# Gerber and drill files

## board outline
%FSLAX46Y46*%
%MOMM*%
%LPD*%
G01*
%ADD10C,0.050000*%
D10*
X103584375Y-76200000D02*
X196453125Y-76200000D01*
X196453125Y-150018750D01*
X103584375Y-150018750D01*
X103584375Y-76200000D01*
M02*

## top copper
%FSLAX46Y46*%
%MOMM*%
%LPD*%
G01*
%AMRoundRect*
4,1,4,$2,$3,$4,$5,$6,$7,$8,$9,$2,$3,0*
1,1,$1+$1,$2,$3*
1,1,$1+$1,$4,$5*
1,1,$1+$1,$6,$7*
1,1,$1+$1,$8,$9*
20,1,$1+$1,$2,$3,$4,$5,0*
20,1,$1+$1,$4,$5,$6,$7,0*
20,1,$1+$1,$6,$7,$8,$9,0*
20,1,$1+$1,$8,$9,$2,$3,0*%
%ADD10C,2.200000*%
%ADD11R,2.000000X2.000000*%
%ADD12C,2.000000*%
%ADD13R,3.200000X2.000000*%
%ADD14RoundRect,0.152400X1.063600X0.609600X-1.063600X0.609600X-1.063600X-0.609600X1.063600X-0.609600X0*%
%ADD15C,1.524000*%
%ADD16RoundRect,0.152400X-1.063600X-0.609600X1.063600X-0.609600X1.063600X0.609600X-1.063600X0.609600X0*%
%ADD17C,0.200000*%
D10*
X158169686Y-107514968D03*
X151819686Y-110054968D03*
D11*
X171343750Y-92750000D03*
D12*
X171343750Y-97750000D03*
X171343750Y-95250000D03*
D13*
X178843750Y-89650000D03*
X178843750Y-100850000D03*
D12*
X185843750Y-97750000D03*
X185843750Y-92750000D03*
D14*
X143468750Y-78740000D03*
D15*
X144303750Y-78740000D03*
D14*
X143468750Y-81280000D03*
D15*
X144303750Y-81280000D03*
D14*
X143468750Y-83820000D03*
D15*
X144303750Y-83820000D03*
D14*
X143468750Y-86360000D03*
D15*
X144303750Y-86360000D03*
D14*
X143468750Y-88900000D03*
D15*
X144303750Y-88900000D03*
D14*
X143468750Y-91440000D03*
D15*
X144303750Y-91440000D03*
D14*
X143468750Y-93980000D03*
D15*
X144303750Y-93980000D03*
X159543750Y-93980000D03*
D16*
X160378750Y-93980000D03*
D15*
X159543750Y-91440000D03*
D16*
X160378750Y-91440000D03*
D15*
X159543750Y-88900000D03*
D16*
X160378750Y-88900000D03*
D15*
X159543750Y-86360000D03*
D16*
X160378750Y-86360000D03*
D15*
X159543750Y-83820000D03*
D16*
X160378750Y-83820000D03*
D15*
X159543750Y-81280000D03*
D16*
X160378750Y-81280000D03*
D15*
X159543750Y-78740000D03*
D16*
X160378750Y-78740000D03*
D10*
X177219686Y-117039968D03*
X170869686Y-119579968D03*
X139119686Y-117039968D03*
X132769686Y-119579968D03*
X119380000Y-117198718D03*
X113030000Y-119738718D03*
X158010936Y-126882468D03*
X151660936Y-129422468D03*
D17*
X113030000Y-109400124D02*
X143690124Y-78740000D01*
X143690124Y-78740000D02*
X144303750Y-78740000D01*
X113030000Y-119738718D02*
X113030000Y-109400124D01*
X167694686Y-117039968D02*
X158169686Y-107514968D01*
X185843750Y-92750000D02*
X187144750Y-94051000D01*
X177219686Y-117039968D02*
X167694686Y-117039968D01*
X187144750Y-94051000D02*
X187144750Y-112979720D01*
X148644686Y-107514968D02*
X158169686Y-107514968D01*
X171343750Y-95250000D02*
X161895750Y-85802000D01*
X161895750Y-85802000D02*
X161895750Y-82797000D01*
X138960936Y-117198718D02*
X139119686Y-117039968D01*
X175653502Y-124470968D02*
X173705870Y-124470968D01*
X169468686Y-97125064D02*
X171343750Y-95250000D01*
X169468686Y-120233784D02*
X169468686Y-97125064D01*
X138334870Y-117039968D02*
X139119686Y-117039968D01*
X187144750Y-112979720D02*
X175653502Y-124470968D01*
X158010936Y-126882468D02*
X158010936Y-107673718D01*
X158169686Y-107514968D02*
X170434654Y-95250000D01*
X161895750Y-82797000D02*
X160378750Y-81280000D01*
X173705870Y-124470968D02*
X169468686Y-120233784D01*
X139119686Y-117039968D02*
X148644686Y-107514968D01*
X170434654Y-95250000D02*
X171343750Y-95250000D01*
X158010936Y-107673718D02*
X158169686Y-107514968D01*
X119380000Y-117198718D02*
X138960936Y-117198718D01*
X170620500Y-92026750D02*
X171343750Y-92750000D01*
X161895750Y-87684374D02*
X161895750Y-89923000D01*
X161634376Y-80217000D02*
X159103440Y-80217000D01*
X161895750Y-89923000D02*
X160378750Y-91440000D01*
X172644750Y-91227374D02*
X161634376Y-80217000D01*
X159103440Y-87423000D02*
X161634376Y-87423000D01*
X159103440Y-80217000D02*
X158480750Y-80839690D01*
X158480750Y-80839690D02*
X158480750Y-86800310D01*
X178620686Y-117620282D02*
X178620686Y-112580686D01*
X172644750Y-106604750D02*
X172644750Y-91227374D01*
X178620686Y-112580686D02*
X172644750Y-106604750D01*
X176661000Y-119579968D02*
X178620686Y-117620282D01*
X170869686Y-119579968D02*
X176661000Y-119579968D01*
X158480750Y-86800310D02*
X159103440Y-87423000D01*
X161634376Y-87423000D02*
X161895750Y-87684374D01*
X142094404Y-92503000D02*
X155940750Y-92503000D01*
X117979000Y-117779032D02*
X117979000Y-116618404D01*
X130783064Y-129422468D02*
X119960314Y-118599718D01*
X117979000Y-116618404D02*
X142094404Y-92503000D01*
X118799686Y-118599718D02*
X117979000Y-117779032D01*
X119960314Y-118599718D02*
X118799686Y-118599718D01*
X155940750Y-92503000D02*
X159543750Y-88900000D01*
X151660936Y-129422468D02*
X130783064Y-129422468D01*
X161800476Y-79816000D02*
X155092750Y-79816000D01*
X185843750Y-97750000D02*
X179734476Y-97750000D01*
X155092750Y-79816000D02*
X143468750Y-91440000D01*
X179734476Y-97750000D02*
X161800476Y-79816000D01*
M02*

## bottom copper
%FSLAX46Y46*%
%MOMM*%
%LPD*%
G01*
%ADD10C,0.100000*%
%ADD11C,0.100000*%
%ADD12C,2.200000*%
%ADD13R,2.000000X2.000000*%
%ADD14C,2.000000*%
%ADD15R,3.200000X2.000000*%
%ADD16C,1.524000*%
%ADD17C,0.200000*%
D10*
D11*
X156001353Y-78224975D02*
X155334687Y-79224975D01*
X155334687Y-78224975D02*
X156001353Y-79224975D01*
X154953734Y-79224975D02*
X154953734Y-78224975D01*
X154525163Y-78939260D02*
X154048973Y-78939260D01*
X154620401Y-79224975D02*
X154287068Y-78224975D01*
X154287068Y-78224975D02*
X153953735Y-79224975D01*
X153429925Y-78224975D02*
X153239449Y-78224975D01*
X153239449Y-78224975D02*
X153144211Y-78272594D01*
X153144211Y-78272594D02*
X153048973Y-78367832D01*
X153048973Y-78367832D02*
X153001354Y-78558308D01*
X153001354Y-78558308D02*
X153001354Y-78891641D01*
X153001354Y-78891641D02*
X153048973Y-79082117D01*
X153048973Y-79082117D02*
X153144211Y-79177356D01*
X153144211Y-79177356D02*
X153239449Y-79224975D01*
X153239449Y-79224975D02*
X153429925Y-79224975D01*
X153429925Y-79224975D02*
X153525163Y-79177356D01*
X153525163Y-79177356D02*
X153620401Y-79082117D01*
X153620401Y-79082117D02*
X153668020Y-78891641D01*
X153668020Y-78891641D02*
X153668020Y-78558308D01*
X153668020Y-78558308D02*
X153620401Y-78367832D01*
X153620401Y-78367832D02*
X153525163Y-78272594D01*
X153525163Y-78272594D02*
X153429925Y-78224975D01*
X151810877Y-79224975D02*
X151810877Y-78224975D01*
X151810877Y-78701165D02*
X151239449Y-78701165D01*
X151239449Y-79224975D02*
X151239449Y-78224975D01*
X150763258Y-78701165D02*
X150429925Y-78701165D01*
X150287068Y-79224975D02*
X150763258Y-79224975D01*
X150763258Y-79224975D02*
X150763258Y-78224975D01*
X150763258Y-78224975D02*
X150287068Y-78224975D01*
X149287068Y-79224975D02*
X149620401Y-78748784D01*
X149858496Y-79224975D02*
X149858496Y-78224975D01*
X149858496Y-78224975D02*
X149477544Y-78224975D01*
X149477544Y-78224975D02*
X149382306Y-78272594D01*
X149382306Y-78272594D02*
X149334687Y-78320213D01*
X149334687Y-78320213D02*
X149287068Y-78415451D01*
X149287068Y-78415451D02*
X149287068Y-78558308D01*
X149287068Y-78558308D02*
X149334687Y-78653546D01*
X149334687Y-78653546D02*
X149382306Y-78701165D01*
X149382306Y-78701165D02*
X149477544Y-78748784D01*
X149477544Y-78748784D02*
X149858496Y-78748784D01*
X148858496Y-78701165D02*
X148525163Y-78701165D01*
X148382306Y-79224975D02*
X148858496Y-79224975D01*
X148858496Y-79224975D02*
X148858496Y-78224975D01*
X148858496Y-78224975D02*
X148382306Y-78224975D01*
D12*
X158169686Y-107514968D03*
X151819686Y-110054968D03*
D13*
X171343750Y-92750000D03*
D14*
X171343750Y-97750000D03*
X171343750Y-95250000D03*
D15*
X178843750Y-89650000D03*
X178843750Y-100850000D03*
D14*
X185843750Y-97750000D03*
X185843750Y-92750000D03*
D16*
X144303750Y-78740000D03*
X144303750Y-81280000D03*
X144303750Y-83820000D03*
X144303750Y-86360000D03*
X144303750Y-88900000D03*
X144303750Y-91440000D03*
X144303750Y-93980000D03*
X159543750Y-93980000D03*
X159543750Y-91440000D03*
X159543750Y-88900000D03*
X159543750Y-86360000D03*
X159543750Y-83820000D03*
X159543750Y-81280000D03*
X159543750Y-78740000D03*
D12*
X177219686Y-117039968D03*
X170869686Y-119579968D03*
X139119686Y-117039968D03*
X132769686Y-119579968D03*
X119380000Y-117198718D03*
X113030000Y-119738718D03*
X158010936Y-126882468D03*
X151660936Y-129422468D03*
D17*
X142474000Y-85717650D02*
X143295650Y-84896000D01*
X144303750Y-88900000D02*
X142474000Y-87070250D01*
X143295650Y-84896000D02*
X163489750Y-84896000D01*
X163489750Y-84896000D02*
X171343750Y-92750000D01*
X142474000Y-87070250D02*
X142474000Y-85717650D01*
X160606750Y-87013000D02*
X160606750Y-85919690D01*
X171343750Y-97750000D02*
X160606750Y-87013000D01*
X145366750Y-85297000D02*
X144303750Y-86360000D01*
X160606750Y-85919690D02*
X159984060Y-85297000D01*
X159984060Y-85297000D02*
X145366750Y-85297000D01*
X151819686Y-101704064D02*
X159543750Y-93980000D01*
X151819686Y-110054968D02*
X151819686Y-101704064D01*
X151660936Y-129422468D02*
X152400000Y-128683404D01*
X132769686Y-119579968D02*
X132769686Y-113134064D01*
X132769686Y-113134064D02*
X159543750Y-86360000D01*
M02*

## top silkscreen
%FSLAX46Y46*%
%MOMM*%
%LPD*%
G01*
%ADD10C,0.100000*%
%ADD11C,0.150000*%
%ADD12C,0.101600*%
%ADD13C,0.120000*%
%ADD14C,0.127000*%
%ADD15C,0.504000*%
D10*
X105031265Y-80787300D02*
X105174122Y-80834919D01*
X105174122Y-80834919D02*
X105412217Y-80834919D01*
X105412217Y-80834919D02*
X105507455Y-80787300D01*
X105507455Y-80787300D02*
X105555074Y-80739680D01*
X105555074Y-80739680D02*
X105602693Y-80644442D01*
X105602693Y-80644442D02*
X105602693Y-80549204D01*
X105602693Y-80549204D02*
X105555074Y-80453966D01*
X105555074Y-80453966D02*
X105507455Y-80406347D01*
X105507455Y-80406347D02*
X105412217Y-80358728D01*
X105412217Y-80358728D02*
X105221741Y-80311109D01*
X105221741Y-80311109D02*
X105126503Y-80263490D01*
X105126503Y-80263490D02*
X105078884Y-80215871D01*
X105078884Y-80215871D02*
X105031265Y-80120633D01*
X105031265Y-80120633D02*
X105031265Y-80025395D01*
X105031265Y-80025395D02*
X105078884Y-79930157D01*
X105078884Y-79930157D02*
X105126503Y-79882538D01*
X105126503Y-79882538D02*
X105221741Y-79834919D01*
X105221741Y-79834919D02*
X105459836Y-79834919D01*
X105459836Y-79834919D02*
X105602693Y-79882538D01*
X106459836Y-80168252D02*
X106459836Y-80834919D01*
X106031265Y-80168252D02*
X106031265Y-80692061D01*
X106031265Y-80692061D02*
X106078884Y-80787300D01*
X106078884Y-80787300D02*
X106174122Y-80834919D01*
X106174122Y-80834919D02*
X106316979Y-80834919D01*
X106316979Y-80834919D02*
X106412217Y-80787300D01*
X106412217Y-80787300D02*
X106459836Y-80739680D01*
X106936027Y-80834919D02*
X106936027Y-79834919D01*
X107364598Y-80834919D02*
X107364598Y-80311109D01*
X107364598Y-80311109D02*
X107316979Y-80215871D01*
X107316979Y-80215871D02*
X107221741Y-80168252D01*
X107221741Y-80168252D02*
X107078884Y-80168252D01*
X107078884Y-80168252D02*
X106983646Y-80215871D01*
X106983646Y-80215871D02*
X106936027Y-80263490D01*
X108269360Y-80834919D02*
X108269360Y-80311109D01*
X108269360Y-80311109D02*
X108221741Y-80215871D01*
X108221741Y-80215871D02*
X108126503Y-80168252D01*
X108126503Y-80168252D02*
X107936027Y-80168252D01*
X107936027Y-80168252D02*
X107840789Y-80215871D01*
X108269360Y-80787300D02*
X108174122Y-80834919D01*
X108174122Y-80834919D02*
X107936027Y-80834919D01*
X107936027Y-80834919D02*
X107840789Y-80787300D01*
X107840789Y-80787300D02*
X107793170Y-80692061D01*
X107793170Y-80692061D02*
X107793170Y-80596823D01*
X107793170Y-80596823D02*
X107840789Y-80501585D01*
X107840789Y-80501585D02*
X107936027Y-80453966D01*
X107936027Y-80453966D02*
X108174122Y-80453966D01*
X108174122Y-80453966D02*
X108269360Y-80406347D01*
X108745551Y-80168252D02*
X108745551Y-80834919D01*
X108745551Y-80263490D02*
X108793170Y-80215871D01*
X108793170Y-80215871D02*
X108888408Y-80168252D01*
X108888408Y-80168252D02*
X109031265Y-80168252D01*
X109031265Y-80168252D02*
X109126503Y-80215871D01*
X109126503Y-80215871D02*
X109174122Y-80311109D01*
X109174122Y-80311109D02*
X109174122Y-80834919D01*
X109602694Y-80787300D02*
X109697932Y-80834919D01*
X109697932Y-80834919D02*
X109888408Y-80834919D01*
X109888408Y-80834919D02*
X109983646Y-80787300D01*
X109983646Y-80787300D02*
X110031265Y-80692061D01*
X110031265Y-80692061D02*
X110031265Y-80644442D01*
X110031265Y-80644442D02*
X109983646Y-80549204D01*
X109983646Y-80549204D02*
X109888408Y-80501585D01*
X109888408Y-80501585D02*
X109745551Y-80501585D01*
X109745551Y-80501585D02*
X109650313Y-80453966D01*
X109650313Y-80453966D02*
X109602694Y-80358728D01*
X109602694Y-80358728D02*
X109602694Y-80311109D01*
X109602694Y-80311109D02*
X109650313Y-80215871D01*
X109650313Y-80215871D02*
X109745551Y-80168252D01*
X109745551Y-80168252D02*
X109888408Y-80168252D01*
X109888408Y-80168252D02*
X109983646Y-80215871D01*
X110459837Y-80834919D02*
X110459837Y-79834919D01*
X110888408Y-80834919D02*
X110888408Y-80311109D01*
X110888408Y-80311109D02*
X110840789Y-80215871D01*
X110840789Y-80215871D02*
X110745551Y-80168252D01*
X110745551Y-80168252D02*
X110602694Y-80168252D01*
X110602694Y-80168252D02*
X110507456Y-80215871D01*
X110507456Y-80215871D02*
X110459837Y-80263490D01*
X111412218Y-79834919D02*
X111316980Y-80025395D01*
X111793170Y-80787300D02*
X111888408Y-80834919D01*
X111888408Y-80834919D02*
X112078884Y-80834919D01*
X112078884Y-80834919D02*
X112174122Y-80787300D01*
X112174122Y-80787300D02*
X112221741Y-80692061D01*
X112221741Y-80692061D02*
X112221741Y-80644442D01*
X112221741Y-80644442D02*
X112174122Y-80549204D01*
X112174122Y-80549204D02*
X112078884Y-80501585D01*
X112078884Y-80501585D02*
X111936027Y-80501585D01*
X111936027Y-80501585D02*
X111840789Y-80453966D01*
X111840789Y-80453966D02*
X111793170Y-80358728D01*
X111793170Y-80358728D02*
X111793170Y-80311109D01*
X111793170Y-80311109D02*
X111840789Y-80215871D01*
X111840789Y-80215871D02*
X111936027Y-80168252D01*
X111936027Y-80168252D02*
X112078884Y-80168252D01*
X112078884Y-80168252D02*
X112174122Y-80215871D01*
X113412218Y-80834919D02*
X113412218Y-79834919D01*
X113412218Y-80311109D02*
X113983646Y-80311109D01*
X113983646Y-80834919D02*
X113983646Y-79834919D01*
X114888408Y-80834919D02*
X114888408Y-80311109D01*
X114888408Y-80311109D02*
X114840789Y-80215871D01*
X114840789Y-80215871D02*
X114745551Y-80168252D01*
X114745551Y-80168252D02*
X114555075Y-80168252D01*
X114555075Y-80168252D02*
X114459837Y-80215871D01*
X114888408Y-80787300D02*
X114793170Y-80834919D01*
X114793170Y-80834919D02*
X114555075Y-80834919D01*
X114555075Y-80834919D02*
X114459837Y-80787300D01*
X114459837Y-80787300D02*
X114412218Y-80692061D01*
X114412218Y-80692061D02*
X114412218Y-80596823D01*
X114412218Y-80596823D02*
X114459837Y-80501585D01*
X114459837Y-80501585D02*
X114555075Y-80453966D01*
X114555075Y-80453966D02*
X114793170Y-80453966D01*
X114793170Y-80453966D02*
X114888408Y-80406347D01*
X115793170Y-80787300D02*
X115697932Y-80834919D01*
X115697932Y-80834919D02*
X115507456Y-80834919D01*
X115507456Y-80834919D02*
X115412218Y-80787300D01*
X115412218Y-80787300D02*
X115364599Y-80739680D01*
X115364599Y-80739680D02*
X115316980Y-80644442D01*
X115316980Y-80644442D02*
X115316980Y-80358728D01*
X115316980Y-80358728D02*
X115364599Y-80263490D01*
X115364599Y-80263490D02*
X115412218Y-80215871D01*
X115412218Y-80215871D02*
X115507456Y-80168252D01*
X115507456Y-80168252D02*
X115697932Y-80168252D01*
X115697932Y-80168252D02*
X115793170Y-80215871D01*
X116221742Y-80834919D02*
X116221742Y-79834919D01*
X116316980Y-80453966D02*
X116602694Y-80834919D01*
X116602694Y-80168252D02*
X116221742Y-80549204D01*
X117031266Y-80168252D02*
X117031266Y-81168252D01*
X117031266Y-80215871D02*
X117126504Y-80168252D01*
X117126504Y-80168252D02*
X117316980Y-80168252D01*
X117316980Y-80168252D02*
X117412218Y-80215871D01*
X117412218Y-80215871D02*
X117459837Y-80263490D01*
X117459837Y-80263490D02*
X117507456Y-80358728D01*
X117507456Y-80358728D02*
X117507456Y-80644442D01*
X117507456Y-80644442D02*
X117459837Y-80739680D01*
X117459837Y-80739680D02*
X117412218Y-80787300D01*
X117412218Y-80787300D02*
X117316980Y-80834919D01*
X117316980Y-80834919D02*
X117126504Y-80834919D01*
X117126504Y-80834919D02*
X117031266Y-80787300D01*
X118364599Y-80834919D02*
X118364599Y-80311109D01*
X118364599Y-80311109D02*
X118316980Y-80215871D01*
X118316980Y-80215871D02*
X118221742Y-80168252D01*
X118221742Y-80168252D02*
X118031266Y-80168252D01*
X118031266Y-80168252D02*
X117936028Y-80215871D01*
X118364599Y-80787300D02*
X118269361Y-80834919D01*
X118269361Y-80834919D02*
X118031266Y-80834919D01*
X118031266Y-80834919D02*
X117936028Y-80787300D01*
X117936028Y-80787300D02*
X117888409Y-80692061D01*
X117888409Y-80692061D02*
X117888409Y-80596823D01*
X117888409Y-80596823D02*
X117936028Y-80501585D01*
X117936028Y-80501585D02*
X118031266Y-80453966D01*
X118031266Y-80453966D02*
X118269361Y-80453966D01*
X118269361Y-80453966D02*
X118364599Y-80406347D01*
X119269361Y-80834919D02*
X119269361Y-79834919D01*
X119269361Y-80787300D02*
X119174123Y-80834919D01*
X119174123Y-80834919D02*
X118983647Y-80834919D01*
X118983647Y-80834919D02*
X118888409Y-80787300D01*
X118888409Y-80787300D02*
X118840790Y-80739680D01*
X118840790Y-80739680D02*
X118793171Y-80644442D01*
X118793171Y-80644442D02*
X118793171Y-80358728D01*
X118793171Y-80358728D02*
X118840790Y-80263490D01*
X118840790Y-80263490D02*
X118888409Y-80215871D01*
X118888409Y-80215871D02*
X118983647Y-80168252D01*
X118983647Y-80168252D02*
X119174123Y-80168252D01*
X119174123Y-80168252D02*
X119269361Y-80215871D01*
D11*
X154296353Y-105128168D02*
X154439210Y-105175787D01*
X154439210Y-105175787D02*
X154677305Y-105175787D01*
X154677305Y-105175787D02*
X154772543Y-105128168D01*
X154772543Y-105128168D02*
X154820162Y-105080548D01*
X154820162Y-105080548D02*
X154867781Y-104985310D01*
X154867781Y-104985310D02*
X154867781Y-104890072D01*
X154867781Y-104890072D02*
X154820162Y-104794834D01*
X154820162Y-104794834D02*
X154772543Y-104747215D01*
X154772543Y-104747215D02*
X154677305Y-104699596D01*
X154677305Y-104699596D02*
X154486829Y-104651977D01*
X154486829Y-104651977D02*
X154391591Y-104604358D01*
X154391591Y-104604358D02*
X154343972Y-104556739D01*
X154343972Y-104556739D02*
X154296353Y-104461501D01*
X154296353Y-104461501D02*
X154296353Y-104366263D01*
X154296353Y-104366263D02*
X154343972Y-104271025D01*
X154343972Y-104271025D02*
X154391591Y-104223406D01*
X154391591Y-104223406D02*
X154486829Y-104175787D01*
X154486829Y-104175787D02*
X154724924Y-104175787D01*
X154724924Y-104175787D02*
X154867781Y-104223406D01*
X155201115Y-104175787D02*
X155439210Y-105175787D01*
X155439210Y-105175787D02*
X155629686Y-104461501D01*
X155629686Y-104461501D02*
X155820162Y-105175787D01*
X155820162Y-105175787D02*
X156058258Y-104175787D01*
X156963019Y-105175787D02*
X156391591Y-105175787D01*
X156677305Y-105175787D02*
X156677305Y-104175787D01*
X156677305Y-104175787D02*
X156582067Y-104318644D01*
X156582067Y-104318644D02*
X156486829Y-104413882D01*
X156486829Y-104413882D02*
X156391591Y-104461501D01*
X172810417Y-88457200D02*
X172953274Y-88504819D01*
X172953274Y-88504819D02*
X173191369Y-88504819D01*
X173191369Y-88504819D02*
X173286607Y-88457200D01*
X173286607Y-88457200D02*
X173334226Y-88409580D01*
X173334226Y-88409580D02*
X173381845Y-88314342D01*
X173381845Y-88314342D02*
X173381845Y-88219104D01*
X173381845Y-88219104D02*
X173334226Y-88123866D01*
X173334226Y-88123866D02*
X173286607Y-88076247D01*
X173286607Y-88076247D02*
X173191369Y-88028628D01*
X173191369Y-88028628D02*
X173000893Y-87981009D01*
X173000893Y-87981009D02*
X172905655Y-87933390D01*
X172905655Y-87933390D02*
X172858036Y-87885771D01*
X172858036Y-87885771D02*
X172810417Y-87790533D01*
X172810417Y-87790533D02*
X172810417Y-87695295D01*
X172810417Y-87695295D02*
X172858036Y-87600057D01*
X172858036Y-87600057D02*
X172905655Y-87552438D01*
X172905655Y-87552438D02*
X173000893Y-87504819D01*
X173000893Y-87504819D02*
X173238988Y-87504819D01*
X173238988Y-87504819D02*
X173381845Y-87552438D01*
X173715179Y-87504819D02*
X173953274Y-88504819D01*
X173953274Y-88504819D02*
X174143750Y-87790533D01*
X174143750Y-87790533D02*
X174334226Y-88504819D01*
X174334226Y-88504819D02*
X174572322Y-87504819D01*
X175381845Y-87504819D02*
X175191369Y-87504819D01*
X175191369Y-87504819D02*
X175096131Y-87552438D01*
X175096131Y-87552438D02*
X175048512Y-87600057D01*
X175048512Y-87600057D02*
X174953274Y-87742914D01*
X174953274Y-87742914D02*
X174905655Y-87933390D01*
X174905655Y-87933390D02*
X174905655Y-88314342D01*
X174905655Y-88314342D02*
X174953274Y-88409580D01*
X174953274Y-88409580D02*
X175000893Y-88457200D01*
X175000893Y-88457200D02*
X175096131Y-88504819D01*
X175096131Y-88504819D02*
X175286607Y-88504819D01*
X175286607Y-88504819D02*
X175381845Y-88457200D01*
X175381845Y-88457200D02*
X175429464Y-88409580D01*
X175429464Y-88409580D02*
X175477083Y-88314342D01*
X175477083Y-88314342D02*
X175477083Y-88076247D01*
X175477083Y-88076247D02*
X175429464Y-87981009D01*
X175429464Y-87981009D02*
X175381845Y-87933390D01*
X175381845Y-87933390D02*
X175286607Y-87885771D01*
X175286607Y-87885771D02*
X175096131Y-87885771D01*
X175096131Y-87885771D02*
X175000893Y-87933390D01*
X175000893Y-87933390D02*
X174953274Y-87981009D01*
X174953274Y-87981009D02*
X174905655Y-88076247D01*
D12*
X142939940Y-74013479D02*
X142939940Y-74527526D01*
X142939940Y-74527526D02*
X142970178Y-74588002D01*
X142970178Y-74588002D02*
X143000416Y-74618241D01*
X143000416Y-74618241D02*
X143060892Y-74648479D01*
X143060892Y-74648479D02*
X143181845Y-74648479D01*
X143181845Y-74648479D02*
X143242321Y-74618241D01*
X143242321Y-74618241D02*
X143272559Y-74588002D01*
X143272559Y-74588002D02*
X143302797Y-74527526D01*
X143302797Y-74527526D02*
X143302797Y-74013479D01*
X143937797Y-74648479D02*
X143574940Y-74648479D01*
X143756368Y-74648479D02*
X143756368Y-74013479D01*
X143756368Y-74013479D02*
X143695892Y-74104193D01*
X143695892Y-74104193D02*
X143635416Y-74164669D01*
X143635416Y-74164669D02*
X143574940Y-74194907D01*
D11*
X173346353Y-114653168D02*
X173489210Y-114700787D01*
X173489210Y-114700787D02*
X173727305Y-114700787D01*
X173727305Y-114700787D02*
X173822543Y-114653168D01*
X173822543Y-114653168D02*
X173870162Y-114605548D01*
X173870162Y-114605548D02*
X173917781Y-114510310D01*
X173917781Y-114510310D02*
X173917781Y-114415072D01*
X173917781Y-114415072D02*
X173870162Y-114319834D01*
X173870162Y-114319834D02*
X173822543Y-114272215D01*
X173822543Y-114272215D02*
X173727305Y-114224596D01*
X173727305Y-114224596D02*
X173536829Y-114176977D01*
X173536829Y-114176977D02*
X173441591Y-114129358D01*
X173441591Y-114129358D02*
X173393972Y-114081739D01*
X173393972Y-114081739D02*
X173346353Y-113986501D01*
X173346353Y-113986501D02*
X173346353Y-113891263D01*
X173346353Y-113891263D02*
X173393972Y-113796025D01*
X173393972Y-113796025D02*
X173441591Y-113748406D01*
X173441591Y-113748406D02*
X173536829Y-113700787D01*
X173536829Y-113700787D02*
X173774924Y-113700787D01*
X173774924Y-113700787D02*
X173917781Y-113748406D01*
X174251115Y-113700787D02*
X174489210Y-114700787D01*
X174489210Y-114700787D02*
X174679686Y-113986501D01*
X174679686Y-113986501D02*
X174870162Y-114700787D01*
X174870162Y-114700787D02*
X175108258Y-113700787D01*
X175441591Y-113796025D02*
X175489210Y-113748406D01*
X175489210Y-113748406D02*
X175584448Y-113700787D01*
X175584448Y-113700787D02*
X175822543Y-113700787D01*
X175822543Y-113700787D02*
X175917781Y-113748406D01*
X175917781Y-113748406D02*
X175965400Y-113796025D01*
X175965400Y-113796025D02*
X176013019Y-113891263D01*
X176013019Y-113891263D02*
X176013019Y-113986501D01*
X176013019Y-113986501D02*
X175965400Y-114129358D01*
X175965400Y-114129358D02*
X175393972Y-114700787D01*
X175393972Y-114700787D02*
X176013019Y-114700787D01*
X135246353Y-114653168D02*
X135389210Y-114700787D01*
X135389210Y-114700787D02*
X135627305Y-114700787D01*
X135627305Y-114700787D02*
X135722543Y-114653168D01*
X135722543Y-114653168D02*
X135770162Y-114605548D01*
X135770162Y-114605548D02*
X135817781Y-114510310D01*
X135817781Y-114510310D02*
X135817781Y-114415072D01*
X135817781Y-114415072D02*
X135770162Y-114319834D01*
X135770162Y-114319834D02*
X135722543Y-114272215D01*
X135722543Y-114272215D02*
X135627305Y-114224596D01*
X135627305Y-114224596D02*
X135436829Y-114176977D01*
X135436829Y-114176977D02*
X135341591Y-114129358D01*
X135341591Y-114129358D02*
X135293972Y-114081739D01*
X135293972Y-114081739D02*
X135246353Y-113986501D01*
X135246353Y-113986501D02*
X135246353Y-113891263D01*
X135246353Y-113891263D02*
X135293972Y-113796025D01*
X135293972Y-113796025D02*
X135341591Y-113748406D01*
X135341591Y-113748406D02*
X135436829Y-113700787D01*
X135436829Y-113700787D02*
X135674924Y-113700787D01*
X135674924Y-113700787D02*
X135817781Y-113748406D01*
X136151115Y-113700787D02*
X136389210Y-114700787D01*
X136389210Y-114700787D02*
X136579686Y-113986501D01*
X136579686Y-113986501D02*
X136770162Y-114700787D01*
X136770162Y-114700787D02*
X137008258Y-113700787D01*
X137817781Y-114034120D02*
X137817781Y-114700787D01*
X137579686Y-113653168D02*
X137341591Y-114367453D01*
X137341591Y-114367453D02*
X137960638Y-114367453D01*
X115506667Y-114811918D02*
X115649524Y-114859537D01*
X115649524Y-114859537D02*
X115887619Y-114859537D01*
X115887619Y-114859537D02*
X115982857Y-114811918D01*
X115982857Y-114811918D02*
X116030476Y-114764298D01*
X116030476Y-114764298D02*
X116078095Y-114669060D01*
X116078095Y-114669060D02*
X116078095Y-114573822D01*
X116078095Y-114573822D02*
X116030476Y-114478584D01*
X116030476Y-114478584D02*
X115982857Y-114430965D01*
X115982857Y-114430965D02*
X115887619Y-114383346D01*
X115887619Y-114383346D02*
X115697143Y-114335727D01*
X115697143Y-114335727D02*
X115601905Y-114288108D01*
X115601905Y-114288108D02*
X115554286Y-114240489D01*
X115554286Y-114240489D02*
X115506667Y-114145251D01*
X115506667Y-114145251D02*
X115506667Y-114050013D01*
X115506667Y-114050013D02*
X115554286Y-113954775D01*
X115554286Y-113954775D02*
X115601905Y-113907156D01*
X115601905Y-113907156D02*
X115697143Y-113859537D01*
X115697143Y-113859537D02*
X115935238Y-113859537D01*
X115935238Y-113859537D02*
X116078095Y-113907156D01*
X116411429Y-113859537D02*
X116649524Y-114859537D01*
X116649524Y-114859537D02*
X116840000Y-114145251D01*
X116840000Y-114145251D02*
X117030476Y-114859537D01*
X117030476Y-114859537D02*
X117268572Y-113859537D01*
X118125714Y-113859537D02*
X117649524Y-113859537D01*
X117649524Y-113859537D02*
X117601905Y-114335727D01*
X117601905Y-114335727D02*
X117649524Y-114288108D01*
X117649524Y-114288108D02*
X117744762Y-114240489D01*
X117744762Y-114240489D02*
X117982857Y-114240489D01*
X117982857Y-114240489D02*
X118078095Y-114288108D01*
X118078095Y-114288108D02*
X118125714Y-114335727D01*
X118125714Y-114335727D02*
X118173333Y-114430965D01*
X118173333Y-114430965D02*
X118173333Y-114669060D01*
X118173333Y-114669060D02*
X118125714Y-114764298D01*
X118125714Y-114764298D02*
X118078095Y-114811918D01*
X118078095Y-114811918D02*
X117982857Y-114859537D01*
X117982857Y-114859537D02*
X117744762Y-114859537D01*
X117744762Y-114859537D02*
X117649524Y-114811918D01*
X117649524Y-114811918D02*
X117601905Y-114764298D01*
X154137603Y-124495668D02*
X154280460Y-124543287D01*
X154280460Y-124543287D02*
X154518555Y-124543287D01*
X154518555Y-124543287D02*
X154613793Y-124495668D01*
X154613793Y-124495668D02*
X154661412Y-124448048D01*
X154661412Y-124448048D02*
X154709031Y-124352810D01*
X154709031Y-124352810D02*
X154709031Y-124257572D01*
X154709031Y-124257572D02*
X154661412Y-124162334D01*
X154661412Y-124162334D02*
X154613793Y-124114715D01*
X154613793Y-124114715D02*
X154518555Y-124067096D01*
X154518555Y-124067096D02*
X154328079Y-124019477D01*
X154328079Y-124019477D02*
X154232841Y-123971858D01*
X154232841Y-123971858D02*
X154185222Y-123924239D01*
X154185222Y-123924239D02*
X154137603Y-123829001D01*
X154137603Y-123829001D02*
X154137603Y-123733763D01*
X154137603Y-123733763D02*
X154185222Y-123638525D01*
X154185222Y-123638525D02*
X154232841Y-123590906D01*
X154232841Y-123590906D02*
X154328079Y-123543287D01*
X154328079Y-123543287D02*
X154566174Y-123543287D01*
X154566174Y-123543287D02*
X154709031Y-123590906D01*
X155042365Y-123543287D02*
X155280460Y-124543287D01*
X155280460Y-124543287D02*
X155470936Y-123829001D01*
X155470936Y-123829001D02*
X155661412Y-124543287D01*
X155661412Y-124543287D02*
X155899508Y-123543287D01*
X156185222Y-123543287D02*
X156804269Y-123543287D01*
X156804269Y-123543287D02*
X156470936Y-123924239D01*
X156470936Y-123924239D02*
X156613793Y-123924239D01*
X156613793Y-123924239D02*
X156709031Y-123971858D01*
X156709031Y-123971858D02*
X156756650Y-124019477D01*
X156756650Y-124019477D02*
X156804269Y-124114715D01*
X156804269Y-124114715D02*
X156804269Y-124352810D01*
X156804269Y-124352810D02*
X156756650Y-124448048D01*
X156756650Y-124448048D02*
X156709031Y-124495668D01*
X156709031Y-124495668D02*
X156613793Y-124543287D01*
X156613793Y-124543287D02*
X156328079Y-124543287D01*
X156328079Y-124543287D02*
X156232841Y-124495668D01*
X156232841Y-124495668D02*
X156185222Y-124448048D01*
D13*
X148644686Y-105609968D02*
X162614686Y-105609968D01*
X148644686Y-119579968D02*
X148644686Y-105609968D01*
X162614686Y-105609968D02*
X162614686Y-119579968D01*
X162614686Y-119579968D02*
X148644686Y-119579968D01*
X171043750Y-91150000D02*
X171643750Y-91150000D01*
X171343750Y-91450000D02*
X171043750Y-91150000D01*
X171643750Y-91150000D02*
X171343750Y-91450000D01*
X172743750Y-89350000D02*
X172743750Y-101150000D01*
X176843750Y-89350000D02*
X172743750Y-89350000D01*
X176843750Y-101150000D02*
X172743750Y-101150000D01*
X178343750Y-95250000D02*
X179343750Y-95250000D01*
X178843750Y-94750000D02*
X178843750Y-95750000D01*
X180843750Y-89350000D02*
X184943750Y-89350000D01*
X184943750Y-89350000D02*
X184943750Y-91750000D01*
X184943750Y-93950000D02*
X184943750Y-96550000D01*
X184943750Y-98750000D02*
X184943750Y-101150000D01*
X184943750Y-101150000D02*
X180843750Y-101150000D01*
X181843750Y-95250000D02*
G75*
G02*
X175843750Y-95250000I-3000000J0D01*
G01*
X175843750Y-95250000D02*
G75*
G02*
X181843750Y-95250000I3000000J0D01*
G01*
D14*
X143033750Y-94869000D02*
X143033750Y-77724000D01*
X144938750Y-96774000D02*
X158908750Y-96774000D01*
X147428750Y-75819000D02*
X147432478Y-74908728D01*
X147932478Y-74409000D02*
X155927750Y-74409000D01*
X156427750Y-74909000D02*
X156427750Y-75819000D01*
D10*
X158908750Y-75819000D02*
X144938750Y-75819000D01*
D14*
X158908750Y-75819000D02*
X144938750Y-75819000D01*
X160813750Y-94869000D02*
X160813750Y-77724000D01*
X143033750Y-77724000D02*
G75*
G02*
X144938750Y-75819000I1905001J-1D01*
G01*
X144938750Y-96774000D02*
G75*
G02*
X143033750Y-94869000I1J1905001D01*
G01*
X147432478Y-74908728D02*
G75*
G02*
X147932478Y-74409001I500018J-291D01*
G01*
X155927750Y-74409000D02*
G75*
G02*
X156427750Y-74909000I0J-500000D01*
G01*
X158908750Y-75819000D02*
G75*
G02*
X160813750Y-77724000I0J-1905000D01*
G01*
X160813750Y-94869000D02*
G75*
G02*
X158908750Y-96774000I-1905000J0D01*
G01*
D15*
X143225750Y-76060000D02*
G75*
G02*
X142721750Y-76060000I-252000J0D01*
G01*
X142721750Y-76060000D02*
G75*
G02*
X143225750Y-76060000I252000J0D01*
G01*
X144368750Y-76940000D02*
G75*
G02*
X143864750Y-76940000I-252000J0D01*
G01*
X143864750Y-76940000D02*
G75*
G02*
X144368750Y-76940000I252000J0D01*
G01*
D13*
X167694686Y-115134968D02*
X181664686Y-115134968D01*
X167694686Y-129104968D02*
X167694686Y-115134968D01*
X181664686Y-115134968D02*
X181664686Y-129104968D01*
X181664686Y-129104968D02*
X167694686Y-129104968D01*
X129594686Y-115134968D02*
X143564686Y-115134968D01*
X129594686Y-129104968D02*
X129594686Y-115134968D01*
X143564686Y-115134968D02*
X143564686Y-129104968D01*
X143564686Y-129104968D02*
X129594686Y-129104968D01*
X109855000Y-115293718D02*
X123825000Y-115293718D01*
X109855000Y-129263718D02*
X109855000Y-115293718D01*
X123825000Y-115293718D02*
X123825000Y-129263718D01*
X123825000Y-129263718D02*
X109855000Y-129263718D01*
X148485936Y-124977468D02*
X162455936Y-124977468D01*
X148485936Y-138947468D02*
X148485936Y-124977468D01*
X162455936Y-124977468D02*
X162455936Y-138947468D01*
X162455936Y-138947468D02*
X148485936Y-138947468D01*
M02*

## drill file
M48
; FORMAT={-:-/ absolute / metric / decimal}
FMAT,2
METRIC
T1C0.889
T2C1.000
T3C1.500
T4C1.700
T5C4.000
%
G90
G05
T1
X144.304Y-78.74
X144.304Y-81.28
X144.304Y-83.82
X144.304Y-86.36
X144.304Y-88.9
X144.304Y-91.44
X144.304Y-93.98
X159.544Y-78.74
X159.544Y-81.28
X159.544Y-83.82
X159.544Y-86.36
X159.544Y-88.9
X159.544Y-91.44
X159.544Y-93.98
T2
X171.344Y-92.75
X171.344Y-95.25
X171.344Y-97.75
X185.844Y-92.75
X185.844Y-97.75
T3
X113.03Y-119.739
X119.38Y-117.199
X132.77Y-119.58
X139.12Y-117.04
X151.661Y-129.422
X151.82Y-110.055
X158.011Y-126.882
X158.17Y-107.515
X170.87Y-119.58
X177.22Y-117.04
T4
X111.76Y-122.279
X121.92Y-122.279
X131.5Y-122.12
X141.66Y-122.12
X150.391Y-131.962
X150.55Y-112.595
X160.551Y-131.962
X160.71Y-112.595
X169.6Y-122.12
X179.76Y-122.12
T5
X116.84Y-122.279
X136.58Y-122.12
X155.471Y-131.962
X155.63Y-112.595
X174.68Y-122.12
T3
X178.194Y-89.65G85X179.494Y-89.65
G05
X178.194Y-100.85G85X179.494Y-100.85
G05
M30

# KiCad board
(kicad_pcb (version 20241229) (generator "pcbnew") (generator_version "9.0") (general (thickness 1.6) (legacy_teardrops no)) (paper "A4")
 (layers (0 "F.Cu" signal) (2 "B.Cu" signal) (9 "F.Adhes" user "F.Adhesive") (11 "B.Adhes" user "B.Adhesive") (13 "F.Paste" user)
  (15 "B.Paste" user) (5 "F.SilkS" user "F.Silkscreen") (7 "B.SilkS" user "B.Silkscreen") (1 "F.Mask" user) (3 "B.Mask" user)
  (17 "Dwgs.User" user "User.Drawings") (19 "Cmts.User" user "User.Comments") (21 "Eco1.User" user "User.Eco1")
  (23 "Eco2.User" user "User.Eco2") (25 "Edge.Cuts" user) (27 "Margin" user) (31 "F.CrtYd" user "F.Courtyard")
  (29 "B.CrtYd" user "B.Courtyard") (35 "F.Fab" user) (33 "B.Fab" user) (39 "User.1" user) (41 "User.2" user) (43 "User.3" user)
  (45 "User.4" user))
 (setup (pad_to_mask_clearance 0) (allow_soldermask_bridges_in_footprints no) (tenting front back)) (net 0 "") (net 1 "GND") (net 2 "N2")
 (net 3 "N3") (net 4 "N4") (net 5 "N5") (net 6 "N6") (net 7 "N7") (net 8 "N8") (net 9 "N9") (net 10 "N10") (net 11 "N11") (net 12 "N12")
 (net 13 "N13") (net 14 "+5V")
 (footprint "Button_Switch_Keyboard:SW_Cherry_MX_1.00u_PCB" (layer "F.Cu") (at 158.169686 107.514968)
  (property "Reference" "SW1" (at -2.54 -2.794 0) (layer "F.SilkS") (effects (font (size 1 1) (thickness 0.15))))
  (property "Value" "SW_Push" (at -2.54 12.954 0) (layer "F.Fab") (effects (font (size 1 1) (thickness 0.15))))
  (fp_line (start -9.525 -1.905) (end 4.445 -1.905) (stroke (width 0.12) (type solid)) (layer "F.SilkS"))
  (fp_line (start -9.525 12.065) (end -9.525 -1.905) (stroke (width 0.12) (type solid)) (layer "F.SilkS"))
  (fp_line (start 4.445 -1.905) (end 4.445 12.065) (stroke (width 0.12) (type solid)) (layer "F.SilkS"))
  (fp_line (start 4.445 12.065) (end -9.525 12.065) (stroke (width 0.12) (type solid)) (layer "F.SilkS"))
  (pad "" np_thru_hole circle (at -7.62 5.08) (size 1.7 1.7) (drill 1.7) (layers "*.Cu" "*.Mask"))
  (pad "" np_thru_hole circle (at -2.54 5.08) (size 4 4) (drill 4) (layers "*.Cu" "*.Mask"))
  (pad "" np_thru_hole circle (at 2.54 5.08) (size 1.7 1.7) (drill 1.7) (layers "*.Cu" "*.Mask"))
  (pad "1" thru_hole circle (at 0 0) (size 2.2 2.2) (drill 1.5) (layers "*.Cu" "*.Mask") (remove_unused_layers no) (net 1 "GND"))
  (pad "2" thru_hole circle (at -6.35 2.54) (size 2.2 2.2) (drill 1.5) (layers "*.Cu" "*.Mask") (remove_unused_layers no) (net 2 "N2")))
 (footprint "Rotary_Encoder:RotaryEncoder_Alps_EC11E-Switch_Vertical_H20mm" (layer "F.Cu") (at 171.34375 92.75)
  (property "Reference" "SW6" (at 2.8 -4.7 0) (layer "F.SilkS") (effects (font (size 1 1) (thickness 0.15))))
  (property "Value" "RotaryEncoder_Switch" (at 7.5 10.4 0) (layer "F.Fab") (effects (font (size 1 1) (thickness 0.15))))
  (fp_line (start -0.3 -1.6) (end 0.3 -1.6) (stroke (width 0.12) (type solid)) (layer "F.SilkS"))
  (fp_line (start 0 -1.3) (end -0.3 -1.6) (stroke (width 0.12) (type solid)) (layer "F.SilkS"))
  (fp_line (start 0.3 -1.6) (end 0 -1.3) (stroke (width 0.12) (type solid)) (layer "F.SilkS"))
  (fp_line (start 1.4 -3.4) (end 1.4 8.4) (stroke (width 0.12) (type solid)) (layer "F.SilkS"))
  (fp_line (start 5.5 -3.4) (end 1.4 -3.4) (stroke (width 0.12) (type solid)) (layer "F.SilkS"))
  (fp_line (start 5.5 8.4) (end 1.4 8.4) (stroke (width 0.12) (type solid)) (layer "F.SilkS"))
  (fp_line (start 7 2.5) (end 8 2.5) (stroke (width 0.12) (type solid)) (layer "F.SilkS"))
  (fp_line (start 7.5 2) (end 7.5 3) (stroke (width 0.12) (type solid)) (layer "F.SilkS"))
  (fp_line (start 9.5 -3.4) (end 13.6 -3.4) (stroke (width 0.12) (type solid)) (layer "F.SilkS"))
  (fp_line (start 13.6 -3.4) (end 13.6 -1) (stroke (width 0.12) (type solid)) (layer "F.SilkS"))
  (fp_line (start 13.6 1.2) (end 13.6 3.8) (stroke (width 0.12) (type solid)) (layer "F.SilkS"))
  (fp_line (start 13.6 6) (end 13.6 8.4) (stroke (width 0.12) (type solid)) (layer "F.SilkS"))
  (fp_line (start 13.6 8.4) (end 9.5 8.4) (stroke (width 0.12) (type solid)) (layer "F.SilkS"))
  (fp_circle (center 7.5 2.5) (end 10.5 2.5) (stroke (width 0.12) (type solid)) (fill no) (layer "F.SilkS"))
  (pad "A" thru_hole rect (at 0 0) (size 2 2) (drill 1) (layers "*.Cu" "*.Mask") (remove_unused_layers no) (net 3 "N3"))
  (pad "B" thru_hole circle (at 0 5) (size 2 2) (drill 1) (layers "*.Cu" "*.Mask") (remove_unused_layers no) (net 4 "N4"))
  (pad "C" thru_hole circle (at 0 2.5) (size 2 2) (drill 1) (layers "*.Cu" "*.Mask") (remove_unused_layers no) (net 1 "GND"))
  (pad "MP" thru_hole rect (at 7.5 -3.1) (size 3.2 2) (drill oval 2.8 1.5) (layers "*.Cu" "*.Mask") (remove_unused_layers no))
  (pad "MP" thru_hole rect (at 7.5 8.1) (size 3.2 2) (drill oval 2.8 1.5) (layers "*.Cu" "*.Mask") (remove_unused_layers no))
  (pad "S1" thru_hole circle (at 14.5 5) (size 2 2) (drill 1) (layers "*.Cu" "*.Mask") (remove_unused_layers no) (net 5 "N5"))
  (pad "S2" thru_hole circle (at 14.5 0) (size 2 2) (drill 1) (layers "*.Cu" "*.Mask") (remove_unused_layers no) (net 1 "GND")))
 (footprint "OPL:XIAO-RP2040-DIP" (layer "F.Cu") (at 151.92375 86.36)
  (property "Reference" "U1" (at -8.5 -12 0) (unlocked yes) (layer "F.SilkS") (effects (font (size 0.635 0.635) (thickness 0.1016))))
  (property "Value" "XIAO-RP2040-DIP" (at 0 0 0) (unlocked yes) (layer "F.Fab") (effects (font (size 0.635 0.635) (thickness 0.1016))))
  (fp_line (start -8.89 8.509) (end -8.89 -8.636) (stroke (width 0.127) (type solid)) (layer "F.SilkS"))
  (fp_line (start -6.985 10.414) (end 6.985 10.414) (stroke (width 0.127) (type solid)) (layer "F.SilkS"))
  (fp_line (start -4.495 -10.541) (end -4.491272 -11.451272) (stroke (width 0.127) (type solid)) (layer "F.SilkS"))
  (fp_line (start -3.991272 -11.951) (end 4.004 -11.951) (stroke (width 0.127) (type solid)) (layer "F.SilkS"))
  (fp_line (start 4.504 -11.451) (end 4.504 -10.541) (stroke (width 0.127) (type solid)) (layer "F.SilkS"))
  (fp_line (start 6.985 -10.541) (end -6.985 -10.541) (stroke (width 0.1) (type solid)) (layer "F.SilkS"))
  (fp_line (start 6.985 -10.541) (end -6.985 -10.541) (stroke (width 0.127) (type solid)) (layer "F.SilkS"))
  (fp_line (start 8.89 8.509) (end 8.89 -8.636) (stroke (width 0.127) (type solid)) (layer "F.SilkS"))
  (fp_arc (start -8.89 -8.636) (mid -8.332038 -9.983038) (end -6.985 -10.541) (stroke (width 0.127) (type solid)) (layer "F.SilkS"))
  (fp_arc (start -6.985 10.414) (mid -8.332038 9.856038) (end -8.89 8.509) (stroke (width 0.127) (type solid)) (layer "F.SilkS"))
  (fp_arc (start -4.491272 -11.451272) (mid -4.344728 -11.80464) (end -3.991272 -11.951) (stroke (width 0.127) (type default))
   (layer "F.SilkS"))
  (fp_arc (start 4.004 -11.951) (mid 4.357553 -11.804553) (end 4.504 -11.451) (stroke (width 0.127) (type default)) (layer "F.SilkS"))
  (fp_arc (start 6.985 -10.541) (mid 8.332038 -9.983038) (end 8.89 -8.636) (stroke (width 0.127) (type solid)) (layer "F.SilkS"))
  (fp_arc (start 8.89 8.509) (mid 8.332038 9.856038) (end 6.985 10.414) (stroke (width 0.127) (type solid)) (layer "F.SilkS"))
  (fp_circle (center -8.95 -10.3) (end -8.95 -10.554) (stroke (width 0.5) (type solid)) (fill yes) (layer "F.SilkS"))
  (fp_circle (center -7.807 -9.42) (end -7.807 -9.674) (stroke (width 0.5) (type solid)) (fill yes) (layer "F.SilkS"))
  (pad "1" smd roundrect (at -8.455 -7.62 180) (size 2.432 1.524) (layers "F.Cu" "F.Mask") (roundrect_rratio 0.1) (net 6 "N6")
   (thermal_bridge_angle 45))
  (pad "1" thru_hole circle (at -7.62 -7.62 180) (size 1.524 1.524) (drill 0.889) (layers "*.Cu" "*.Mask") (remove_unused_layers no)
   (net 6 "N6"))
  (pad "2" smd roundrect (at -8.455 -5.08 180) (size 2.432 1.524) (layers "F.Cu" "F.Mask") (roundrect_rratio 0.1) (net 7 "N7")
   (thermal_bridge_angle 45))
  (pad "2" thru_hole circle (at -7.62 -5.08 180) (size 1.524 1.524) (drill 0.889) (layers "*.Cu" "*.Mask") (remove_unused_layers no)
   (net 7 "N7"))
  (pad "3" smd roundrect (at -8.455 -2.54 180) (size 2.432 1.524) (layers "F.Cu" "F.Mask") (roundrect_rratio 0.1) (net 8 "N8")
   (thermal_bridge_angle 45))
  (pad "3" thru_hole circle (at -7.62 -2.54 180) (size 1.524 1.524) (drill 0.889) (layers "*.Cu" "*.Mask") (remove_unused_layers no)
   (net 8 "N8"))
  (pad "4" smd roundrect (at -8.455 0 180) (size 2.432 1.524) (layers "F.Cu" "F.Mask") (roundrect_rratio 0.1) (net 4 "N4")
   (thermal_bridge_angle 45))
  (pad "4" thru_hole circle (at -7.62 0 180) (size 1.524 1.524) (drill 0.889) (layers "*.Cu" "*.Mask") (remove_unused_layers no)
   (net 4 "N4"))
  (pad "5" smd roundrect (at -8.455 2.54 180) (size 2.432 1.524) (layers "F.Cu" "F.Mask") (roundrect_rratio 0.1) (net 3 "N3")
   (thermal_bridge_angle 45))
  (pad "5" thru_hole circle (at -7.62 2.54 180) (size 1.524 1.524) (drill 0.889) (layers "*.Cu" "*.Mask") (remove_unused_layers no)
   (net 3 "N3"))
  (pad "6" smd roundrect (at -8.455 5.08 180) (size 2.432 1.524) (layers "F.Cu" "F.Mask") (roundrect_rratio 0.1) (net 5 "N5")
   (thermal_bridge_angle 45))
  (pad "6" thru_hole circle (at -7.62 5.08 180) (size 1.524 1.524) (drill 0.889) (layers "*.Cu" "*.Mask") (remove_unused_layers no)
   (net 5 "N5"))
  (pad "7" smd roundrect (at -8.455 7.62 180) (size 2.432 1.524) (layers "F.Cu" "F.Mask") (roundrect_rratio 0.1) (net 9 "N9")
   (thermal_bridge_angle 45))
  (pad "7" thru_hole circle (at -7.62 7.62 180) (size 1.524 1.524) (drill 0.889) (layers "*.Cu" "*.Mask") (remove_unused_layers no)
   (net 9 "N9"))
  (pad "8" thru_hole circle (at 7.62 7.62) (size 1.524 1.524) (drill 0.889) (layers "*.Cu" "*.Mask") (remove_unused_layers no) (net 2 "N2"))
  (pad "8" smd roundrect (at 8.455 7.62) (size 2.432 1.524) (layers "F.Cu" "F.Mask") (roundrect_rratio 0.1) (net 2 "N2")
   (thermal_bridge_angle 45))
  (pad "9" thru_hole circle (at 7.62 5.08) (size 1.524 1.524) (drill 0.889) (layers "*.Cu" "*.Mask") (remove_unused_layers no)
   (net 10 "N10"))
  (pad "9" smd roundrect (at 8.455 5.08) (size 2.432 1.524) (layers "F.Cu" "F.Mask") (roundrect_rratio 0.1) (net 10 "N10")
   (thermal_bridge_angle 45))
  (pad "10" thru_hole circle (at 7.62 2.54) (size 1.524 1.524) (drill 0.889) (layers "*.Cu" "*.Mask") (remove_unused_layers no)
   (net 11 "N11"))
  (pad "10" smd roundrect (at 8.455 2.54) (size 2.432 1.524) (layers "F.Cu" "F.Mask") (roundrect_rratio 0.1) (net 11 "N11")
   (thermal_bridge_angle 45))
  (pad "11" thru_hole circle (at 7.62 0) (size 1.524 1.524) (drill 0.889) (layers "*.Cu" "*.Mask") (remove_unused_layers no) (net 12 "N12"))
  (pad "11" smd roundrect (at 8.455 0) (size 2.432 1.524) (layers "F.Cu" "F.Mask") (roundrect_rratio 0.1) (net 12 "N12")
   (thermal_bridge_angle 45))
  (pad "12" thru_hole circle (at 7.62 -2.54) (size 1.524 1.524) (drill 0.889) (layers "*.Cu" "*.Mask") (remove_unused_layers no)
   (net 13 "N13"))
  (pad "12" smd roundrect (at 8.455 -2.54) (size 2.432 1.524) (layers "F.Cu" "F.Mask") (roundrect_rratio 0.1) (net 13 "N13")
   (thermal_bridge_angle 45))
  (pad "13" thru_hole circle (at 7.62 -5.08) (size 1.524 1.524) (drill 0.889) (layers "*.Cu" "*.Mask") (remove_unused_layers no)
   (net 1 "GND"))
  (pad "13" smd roundrect (at 8.455 -5.08) (size 2.432 1.524) (layers "F.Cu" "F.Mask") (roundrect_rratio 0.1) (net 1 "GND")
   (thermal_bridge_angle 45))
  (pad "14" thru_hole circle (at 7.62 -7.62) (size 1.524 1.524) (drill 0.889) (layers "*.Cu" "*.Mask") (remove_unused_layers no)
   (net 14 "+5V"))
  (pad "14" smd roundrect (at 8.455 -7.62) (size 2.432 1.524) (layers "F.Cu" "F.Mask") (roundrect_rratio 0.1) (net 14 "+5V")
   (thermal_bridge_angle 45)))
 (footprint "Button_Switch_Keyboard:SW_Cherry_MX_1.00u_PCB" (layer "F.Cu") (at 177.219686 117.039968)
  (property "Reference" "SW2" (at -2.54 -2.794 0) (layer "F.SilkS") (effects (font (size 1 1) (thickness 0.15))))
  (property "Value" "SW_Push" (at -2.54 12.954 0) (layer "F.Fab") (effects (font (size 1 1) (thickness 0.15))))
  (fp_line (start -9.525 -1.905) (end 4.445 -1.905) (stroke (width 0.12) (type solid)) (layer "F.SilkS"))
  (fp_line (start -9.525 12.065) (end -9.525 -1.905) (stroke (width 0.12) (type solid)) (layer "F.SilkS"))
  (fp_line (start 4.445 -1.905) (end 4.445 12.065) (stroke (width 0.12) (type solid)) (layer "F.SilkS"))
  (fp_line (start 4.445 12.065) (end -9.525 12.065) (stroke (width 0.12) (type solid)) (layer "F.SilkS"))
  (pad "" np_thru_hole circle (at -7.62 5.08) (size 1.7 1.7) (drill 1.7) (layers "*.Cu" "*.Mask"))
  (pad "" np_thru_hole circle (at -2.54 5.08) (size 4 4) (drill 4) (layers "*.Cu" "*.Mask"))
  (pad "" np_thru_hole circle (at 2.54 5.08) (size 1.7 1.7) (drill 1.7) (layers "*.Cu" "*.Mask"))
  (pad "1" thru_hole circle (at 0 0) (size 2.2 2.2) (drill 1.5) (layers "*.Cu" "*.Mask") (remove_unused_layers no) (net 1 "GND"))
  (pad "2" thru_hole circle (at -6.35 2.54) (size 2.2 2.2) (drill 1.5) (layers "*.Cu" "*.Mask") (remove_unused_layers no) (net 10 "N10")))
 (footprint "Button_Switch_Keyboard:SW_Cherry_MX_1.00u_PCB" (layer "F.Cu") (at 139.119686 117.039968)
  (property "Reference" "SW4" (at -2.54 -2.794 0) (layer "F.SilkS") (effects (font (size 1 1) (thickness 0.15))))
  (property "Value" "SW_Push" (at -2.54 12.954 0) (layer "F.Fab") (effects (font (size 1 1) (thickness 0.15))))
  (fp_line (start -9.525 -1.905) (end 4.445 -1.905) (stroke (width 0.12) (type solid)) (layer "F.SilkS"))
  (fp_line (start -9.525 12.065) (end -9.525 -1.905) (stroke (width 0.12) (type solid)) (layer "F.SilkS"))
  (fp_line (start 4.445 -1.905) (end 4.445 12.065) (stroke (width 0.12) (type solid)) (layer "F.SilkS"))
  (fp_line (start 4.445 12.065) (end -9.525 12.065) (stroke (width 0.12) (type solid)) (layer "F.SilkS"))
  (pad "" np_thru_hole circle (at -7.62 5.08) (size 1.7 1.7) (drill 1.7) (layers "*.Cu" "*.Mask"))
  (pad "" np_thru_hole circle (at -2.54 5.08) (size 4 4) (drill 4) (layers "*.Cu" "*.Mask"))
  (pad "" np_thru_hole circle (at 2.54 5.08) (size 1.7 1.7) (drill 1.7) (layers "*.Cu" "*.Mask"))
  (pad "1" thru_hole circle (at 0 0) (size 2.2 2.2) (drill 1.5) (layers "*.Cu" "*.Mask") (remove_unused_layers no) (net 1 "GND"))
  (pad "2" thru_hole circle (at -6.35 2.54) (size 2.2 2.2) (drill 1.5) (layers "*.Cu" "*.Mask") (remove_unused_layers no) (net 12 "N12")))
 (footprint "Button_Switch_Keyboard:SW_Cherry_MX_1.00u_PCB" (layer "F.Cu") (at 119.38 117.198718)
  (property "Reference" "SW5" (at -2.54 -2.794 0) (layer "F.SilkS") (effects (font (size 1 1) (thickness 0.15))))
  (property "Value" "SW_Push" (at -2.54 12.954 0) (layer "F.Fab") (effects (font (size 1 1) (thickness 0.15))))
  (fp_line (start -9.525 -1.905) (end 4.445 -1.905) (stroke (width 0.12) (type solid)) (layer "F.SilkS"))
  (fp_line (start -9.525 12.065) (end -9.525 -1.905) (stroke (width 0.12) (type solid)) (layer "F.SilkS"))
  (fp_line (start 4.445 -1.905) (end 4.445 12.065) (stroke (width 0.12) (type solid)) (layer "F.SilkS"))
  (fp_line (start 4.445 12.065) (end -9.525 12.065) (stroke (width 0.12) (type solid)) (layer "F.SilkS"))
  (pad "" np_thru_hole circle (at -7.62 5.08) (size 1.7 1.7) (drill 1.7) (layers "*.Cu" "*.Mask"))
  (pad "" np_thru_hole circle (at -2.54 5.08) (size 4 4) (drill 4) (layers "*.Cu" "*.Mask"))
  (pad "" np_thru_hole circle (at 2.54 5.08) (size 1.7 1.7) (drill 1.7) (layers "*.Cu" "*.Mask"))
  (pad "1" thru_hole circle (at 0 0) (size 2.2 2.2) (drill 1.5) (layers "*.Cu" "*.Mask") (remove_unused_layers no) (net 1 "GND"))
  (pad "2" thru_hole circle (at -6.35 2.54) (size 2.2 2.2) (drill 1.5) (layers "*.Cu" "*.Mask") (remove_unused_layers no) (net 6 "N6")))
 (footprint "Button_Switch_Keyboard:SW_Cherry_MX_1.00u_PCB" (layer "F.Cu") (at 158.010936 126.882468)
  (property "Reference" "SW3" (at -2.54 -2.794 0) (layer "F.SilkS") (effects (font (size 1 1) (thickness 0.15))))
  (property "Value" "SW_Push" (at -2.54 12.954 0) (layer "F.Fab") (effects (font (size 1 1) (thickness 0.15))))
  (fp_line (start -9.525 -1.905) (end 4.445 -1.905) (stroke (width 0.12) (type solid)) (layer "F.SilkS"))
  (fp_line (start -9.525 12.065) (end -9.525 -1.905) (stroke (width 0.12) (type solid)) (layer "F.SilkS"))
  (fp_line (start 4.445 -1.905) (end 4.445 12.065) (stroke (width 0.12) (type solid)) (layer "F.SilkS"))
  (fp_line (start 4.445 12.065) (end -9.525 12.065) (stroke (width 0.12) (type solid)) (layer "F.SilkS"))
  (pad "" np_thru_hole circle (at -7.62 5.08) (size 1.7 1.7) (drill 1.7) (layers "*.Cu" "*.Mask"))
  (pad "" np_thru_hole circle (at -2.54 5.08) (size 4 4) (drill 4) (layers "*.Cu" "*.Mask"))
  (pad "" np_thru_hole circle (at 2.54 5.08) (size 1.7 1.7) (drill 1.7) (layers "*.Cu" "*.Mask"))
  (pad "1" thru_hole circle (at 0 0) (size 2.2 2.2) (drill 1.5) (layers "*.Cu" "*.Mask") (remove_unused_layers no) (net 1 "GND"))
  (pad "2" thru_hole circle (at -6.35 2.54) (size 2.2 2.2) (drill 1.5) (layers "*.Cu" "*.Mask") (remove_unused_layers no) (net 11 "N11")))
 (gr_rect (start 103.584375 76.2) (end 196.453125 150.01875) (stroke (width 0.05) (type default)) (fill no) (layer "Edge.Cuts"))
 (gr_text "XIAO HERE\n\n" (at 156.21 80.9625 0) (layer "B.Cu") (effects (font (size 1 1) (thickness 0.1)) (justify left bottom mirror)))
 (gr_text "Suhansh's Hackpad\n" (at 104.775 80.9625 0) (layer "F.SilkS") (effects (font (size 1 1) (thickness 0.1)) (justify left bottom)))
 (segment (start 113.03 109.400124) (end 143.690124 78.74) (width 0.2) (layer "F.Cu") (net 6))
 (segment (start 143.690124 78.74) (end 144.30375 78.74) (width 0.2) (layer "F.Cu") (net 6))
 (segment (start 113.03 119.738718) (end 113.03 109.400124) (width 0.2) (layer "F.Cu") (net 6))
 (segment (start 167.694686 117.039968) (end 158.169686 107.514968) (width 0.2) (layer "F.Cu") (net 1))
 (segment (start 185.84375 92.75) (end 187.14475 94.051) (width 0.2) (layer "F.Cu") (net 1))
 (segment (start 177.219686 117.039968) (end 167.694686 117.039968) (width 0.2) (layer "F.Cu") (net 1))
 (segment (start 187.14475 94.051) (end 187.14475 112.97972) (width 0.2) (layer "F.Cu") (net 1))
 (segment (start 148.644686 107.514968) (end 158.169686 107.514968) (width 0.2) (layer "F.Cu") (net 1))
 (segment (start 171.34375 95.25) (end 161.89575 85.802) (width 0.2) (layer "F.Cu") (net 1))
 (segment (start 161.89575 85.802) (end 161.89575 82.797) (width 0.2) (layer "F.Cu") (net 1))
 (segment (start 138.960936 117.198718) (end 139.119686 117.039968) (width 0.2) (layer "F.Cu") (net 1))
 (segment (start 175.653502 124.470968) (end 173.70587 124.470968) (width 0.2) (layer "F.Cu") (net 1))
 (segment (start 169.468686 97.125064) (end 171.34375 95.25) (width 0.2) (layer "F.Cu") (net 1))
 (segment (start 169.468686 120.233784) (end 169.468686 97.125064) (width 0.2) (layer "F.Cu") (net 1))
 (segment (start 138.33487 117.039968) (end 139.119686 117.039968) (width 0.2) (layer "F.Cu") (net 1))
 (segment (start 187.14475 112.97972) (end 175.653502 124.470968) (width 0.2) (layer "F.Cu") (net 1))
 (segment (start 158.010936 126.882468) (end 158.010936 107.673718) (width 0.2) (layer "F.Cu") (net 1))
 (segment (start 158.169686 107.514968) (end 170.434654 95.25) (width 0.2) (layer "F.Cu") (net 1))
 (segment (start 161.89575 82.797) (end 160.37875 81.28) (width 0.2) (layer "F.Cu") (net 1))
 (segment (start 173.70587 124.470968) (end 169.468686 120.233784) (width 0.2) (layer "F.Cu") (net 1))
 (segment (start 139.119686 117.039968) (end 148.644686 107.514968) (width 0.2) (layer "F.Cu") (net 1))
 (segment (start 170.434654 95.25) (end 171.34375 95.25) (width 0.2) (layer "F.Cu") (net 1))
 (segment (start 158.010936 107.673718) (end 158.169686 107.514968) (width 0.2) (layer "F.Cu") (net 1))
 (segment (start 119.38 117.198718) (end 138.960936 117.198718) (width 0.2) (layer "F.Cu") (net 1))
 (segment (start 170.6205 92.02675) (end 171.34375 92.75) (width 0.2) (layer "F.Cu") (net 3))
 (segment (start 142.474 85.71765) (end 143.29565 84.896) (width 0.2) (layer "B.Cu") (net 3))
 (segment (start 144.30375 88.9) (end 142.474 87.07025) (width 0.2) (layer "B.Cu") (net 3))
 (segment (start 143.29565 84.896) (end 163.48975 84.896) (width 0.2) (layer "B.Cu") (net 3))
 (segment (start 163.48975 84.896) (end 171.34375 92.75) (width 0.2) (layer "B.Cu") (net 3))
 (segment (start 142.474 87.07025) (end 142.474 85.71765) (width 0.2) (layer "B.Cu") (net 3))
 (segment (start 160.60675 87.013) (end 160.60675 85.91969) (width 0.2) (layer "B.Cu") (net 4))
 (segment (start 171.34375 97.75) (end 160.60675 87.013) (width 0.2) (layer "B.Cu") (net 4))
 (segment (start 145.36675 85.297) (end 144.30375 86.36) (width 0.2) (layer "B.Cu") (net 4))
 (segment (start 160.60675 85.91969) (end 159.98406 85.297) (width 0.2) (layer "B.Cu") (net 4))
 (segment (start 159.98406 85.297) (end 145.36675 85.297) (width 0.2) (layer "B.Cu") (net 4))
 (segment (start 151.819686 101.704064) (end 159.54375 93.98) (width 0.2) (layer "B.Cu") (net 2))
 (segment (start 151.819686 110.054968) (end 151.819686 101.704064) (width 0.2) (layer "B.Cu") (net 2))
 (segment (start 161.89575 87.684374) (end 161.89575 89.923) (width 0.2) (layer "F.Cu") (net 10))
 (segment (start 161.634376 80.217) (end 159.10344 80.217) (width 0.2) (layer "F.Cu") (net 10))
 (segment (start 161.89575 89.923) (end 160.37875 91.44) (width 0.2) (layer "F.Cu") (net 10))
 (segment (start 172.64475 91.227374) (end 161.634376 80.217) (width 0.2) (layer "F.Cu") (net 10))
 (segment (start 159.10344 87.423) (end 161.634376 87.423) (width 0.2) (layer "F.Cu") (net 10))
 (segment (start 159.10344 80.217) (end 158.48075 80.83969) (width 0.2) (layer "F.Cu") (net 10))
 (segment (start 158.48075 80.83969) (end 158.48075 86.80031) (width 0.2) (layer "F.Cu") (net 10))
 (segment (start 178.620686 117.620282) (end 178.620686 112.580686) (width 0.2) (layer "F.Cu") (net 10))
 (segment (start 172.64475 106.60475) (end 172.64475 91.227374) (width 0.2) (layer "F.Cu") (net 10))
 (segment (start 178.620686 112.580686) (end 172.64475 106.60475) (width 0.2) (layer "F.Cu") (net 10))
 (segment (start 176.661 119.579968) (end 178.620686 117.620282) (width 0.2) (layer "F.Cu") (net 10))
 (segment (start 170.869686 119.579968) (end 176.661 119.579968) (width 0.2) (layer "F.Cu") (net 10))
 (segment (start 158.48075 86.80031) (end 159.10344 87.423) (width 0.2) (layer "F.Cu") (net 10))
 (segment (start 161.634376 87.423) (end 161.89575 87.684374) (width 0.2) (layer "F.Cu") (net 10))
 (segment (start 142.094404 92.503) (end 155.94075 92.503) (width 0.2) (layer "F.Cu") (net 11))
 (segment (start 117.979 117.779032) (end 117.979 116.618404) (width 0.2) (layer "F.Cu") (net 11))
 (segment (start 130.783064 129.422468) (end 119.960314 118.599718) (width 0.2) (layer "F.Cu") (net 11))
 (segment (start 117.979 116.618404) (end 142.094404 92.503) (width 0.2) (layer "F.Cu") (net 11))
 (segment (start 118.799686 118.599718) (end 117.979 117.779032) (width 0.2) (layer "F.Cu") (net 11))
 (segment (start 119.960314 118.599718) (end 118.799686 118.599718) (width 0.2) (layer "F.Cu") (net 11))
 (segment (start 155.94075 92.503) (end 159.54375 88.9) (width 0.2) (layer "F.Cu") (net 11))
 (segment (start 151.660936 129.422468) (end 130.783064 129.422468) (width 0.2) (layer "F.Cu") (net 11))
 (segment (start 151.660936 129.422468) (end 152.4 128.683404) (width 0.2) (layer "B.Cu") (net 11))
 (segment (start 132.769686 119.579968) (end 132.769686 113.134064) (width 0.2) (layer "B.Cu") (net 12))
 (segment (start 132.769686 113.134064) (end 159.54375 86.36) (width 0.2) (layer "B.Cu") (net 12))
 (segment (start 161.800476 79.816) (end 155.09275 79.816) (width 0.2) (layer "F.Cu") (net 5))
 (segment (start 185.84375 97.75) (end 179.734476 97.75) (width 0.2) (layer "F.Cu") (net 5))
 (segment (start 155.09275 79.816) (end 143.46875 91.44) (width 0.2) (layer "F.Cu") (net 5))
 (segment (start 179.734476 97.75) (end 161.800476 79.816) (width 0.2) (layer "F.Cu") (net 5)))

